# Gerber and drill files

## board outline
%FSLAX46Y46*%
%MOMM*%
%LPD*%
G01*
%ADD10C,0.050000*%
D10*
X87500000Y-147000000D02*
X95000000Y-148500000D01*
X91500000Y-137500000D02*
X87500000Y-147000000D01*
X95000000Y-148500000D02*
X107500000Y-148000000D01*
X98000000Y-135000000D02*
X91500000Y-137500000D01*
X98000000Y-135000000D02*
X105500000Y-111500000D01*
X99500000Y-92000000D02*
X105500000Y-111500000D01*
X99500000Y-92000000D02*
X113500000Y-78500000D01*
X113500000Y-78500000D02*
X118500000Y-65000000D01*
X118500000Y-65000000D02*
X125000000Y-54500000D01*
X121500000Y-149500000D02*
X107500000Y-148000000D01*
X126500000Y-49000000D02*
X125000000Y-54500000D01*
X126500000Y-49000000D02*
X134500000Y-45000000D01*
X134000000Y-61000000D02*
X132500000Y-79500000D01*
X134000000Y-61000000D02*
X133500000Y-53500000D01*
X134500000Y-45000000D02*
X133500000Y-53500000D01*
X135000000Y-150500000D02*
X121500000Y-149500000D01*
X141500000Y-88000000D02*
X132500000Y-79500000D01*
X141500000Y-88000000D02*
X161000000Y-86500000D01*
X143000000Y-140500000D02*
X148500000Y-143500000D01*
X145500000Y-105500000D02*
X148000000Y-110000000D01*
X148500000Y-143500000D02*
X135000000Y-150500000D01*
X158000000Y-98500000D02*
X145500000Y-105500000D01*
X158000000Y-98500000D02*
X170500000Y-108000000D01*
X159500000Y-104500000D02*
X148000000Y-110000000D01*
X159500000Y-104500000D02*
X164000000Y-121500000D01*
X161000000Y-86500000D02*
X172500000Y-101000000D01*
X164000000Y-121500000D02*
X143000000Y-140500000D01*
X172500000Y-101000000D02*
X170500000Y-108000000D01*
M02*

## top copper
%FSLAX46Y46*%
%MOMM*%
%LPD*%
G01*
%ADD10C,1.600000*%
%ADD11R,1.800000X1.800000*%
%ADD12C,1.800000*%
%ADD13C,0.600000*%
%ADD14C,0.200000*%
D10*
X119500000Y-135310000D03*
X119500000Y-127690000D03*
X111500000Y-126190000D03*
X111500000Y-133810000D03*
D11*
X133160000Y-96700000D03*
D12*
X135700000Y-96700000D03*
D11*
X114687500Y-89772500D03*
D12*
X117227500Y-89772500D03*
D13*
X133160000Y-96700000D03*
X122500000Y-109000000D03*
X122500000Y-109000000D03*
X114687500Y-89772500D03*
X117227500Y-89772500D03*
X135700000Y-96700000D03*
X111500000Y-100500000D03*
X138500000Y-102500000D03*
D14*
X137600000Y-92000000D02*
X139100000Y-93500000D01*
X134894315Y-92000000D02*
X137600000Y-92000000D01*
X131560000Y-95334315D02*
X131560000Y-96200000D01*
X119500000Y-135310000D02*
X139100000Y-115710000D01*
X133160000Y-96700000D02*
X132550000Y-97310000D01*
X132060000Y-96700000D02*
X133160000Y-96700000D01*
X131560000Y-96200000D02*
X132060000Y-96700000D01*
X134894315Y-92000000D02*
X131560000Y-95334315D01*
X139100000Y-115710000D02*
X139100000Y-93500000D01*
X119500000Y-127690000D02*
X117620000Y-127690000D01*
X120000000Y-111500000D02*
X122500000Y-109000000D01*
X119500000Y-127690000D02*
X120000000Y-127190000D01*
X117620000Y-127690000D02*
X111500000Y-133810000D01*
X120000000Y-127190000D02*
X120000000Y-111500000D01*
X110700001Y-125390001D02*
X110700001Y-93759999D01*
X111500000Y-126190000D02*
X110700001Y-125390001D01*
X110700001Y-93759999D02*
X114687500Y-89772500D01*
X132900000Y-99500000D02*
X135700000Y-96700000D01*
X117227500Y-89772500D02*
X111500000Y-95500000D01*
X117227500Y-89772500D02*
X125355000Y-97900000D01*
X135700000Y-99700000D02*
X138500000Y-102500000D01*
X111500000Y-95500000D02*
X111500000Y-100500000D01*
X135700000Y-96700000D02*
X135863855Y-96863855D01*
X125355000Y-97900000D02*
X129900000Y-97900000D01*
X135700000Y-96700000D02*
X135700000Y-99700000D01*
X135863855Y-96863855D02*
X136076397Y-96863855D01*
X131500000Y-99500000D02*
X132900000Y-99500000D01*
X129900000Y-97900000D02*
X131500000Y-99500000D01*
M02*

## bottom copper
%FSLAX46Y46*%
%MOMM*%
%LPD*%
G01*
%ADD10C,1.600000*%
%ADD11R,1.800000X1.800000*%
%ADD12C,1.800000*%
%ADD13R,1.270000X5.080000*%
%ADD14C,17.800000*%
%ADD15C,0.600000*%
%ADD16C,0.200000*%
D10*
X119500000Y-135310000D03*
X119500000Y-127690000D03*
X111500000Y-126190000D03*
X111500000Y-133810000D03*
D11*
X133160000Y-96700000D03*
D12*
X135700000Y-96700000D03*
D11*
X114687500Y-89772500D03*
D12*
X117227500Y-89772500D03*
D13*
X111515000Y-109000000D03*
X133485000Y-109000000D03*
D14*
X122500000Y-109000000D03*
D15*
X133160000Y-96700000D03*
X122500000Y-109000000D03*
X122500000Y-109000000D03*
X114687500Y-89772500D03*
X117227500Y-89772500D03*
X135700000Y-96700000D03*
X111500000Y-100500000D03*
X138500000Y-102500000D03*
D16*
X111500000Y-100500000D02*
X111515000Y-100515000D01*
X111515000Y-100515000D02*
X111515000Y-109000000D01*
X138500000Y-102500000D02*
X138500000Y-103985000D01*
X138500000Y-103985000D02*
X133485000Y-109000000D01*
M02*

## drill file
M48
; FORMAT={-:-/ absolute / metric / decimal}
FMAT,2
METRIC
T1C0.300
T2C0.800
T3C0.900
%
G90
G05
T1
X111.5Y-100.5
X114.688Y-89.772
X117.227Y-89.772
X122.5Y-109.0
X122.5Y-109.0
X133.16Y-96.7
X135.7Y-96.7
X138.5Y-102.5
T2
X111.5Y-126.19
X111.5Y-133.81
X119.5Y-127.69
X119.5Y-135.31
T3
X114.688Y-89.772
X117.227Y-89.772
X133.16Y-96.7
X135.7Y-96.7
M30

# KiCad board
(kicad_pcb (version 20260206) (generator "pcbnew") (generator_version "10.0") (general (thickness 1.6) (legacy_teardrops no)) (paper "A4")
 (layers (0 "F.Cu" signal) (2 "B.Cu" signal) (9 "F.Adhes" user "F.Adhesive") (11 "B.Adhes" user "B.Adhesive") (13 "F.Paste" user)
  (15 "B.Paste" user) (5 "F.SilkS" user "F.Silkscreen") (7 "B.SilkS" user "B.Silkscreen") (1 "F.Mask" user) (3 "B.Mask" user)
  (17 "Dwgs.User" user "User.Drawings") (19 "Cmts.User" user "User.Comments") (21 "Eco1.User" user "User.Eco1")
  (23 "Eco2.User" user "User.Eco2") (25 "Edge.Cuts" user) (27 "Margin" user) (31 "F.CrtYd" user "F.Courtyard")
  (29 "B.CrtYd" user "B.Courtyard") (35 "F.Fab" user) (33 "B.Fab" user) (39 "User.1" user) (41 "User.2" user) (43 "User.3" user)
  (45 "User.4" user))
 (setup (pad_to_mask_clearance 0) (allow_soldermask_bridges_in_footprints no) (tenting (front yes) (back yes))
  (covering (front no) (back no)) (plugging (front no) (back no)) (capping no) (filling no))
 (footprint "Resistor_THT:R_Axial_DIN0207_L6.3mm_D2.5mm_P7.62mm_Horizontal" (layer "F.Cu") (at 119.5 135.31 90)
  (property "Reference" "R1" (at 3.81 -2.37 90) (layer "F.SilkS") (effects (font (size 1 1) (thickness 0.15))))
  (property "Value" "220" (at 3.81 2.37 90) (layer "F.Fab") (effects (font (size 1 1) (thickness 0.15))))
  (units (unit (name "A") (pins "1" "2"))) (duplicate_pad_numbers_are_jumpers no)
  (pad "1" thru_hole circle (at 0 0 90) (size 1.6 1.6) (drill 0.8) (layers "*.Cu" "*.Mask") (remove_unused_layers no) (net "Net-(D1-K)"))
  (pad "2" thru_hole circle (at 7.62 0 90) (size 1.6 1.6) (drill 0.8) (layers "*.Cu" "*.Mask") (remove_unused_layers no) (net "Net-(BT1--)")))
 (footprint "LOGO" (layer "F.Cu") (at 130 97.5)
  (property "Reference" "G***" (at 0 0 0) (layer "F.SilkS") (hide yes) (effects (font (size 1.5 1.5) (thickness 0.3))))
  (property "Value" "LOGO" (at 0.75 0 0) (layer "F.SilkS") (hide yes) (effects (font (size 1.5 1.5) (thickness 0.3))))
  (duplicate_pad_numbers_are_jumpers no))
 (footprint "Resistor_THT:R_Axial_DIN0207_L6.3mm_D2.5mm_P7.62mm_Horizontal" (layer "F.Cu") (at 111.5 126.19 -90)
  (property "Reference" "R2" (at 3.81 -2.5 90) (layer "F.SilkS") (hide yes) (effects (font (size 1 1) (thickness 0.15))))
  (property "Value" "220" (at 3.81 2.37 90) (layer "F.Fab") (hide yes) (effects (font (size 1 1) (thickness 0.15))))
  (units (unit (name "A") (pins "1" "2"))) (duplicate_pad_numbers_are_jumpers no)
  (pad "1" thru_hole circle (at 0 0 270) (size 1.6 1.6) (drill 0.8) (layers "*.Cu" "*.Mask") (remove_unused_layers no) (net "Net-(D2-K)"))
  (pad "2" thru_hole circle (at 7.62 0 270) (size 1.6 1.6) (drill 0.8) (layers "*.Cu" "*.Mask") (remove_unused_layers no)
   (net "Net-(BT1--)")))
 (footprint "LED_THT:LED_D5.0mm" (layer "F.Cu") (at 133.16 96.7)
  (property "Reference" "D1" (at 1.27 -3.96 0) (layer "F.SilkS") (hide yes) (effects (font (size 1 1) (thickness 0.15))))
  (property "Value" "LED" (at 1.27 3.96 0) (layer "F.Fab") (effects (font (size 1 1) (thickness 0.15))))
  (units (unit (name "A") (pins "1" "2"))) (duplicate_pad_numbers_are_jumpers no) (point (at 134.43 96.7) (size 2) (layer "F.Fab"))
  (pad "1" thru_hole rect (at 0 0) (size 1.8 1.8) (drill 0.9) (layers "*.Cu" "*.Mask") (remove_unused_layers no) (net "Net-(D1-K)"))
  (pad "2" thru_hole circle (at 2.54 0) (size 1.8 1.8) (drill 0.9) (layers "*.Cu" "*.Mask") (remove_unused_layers no) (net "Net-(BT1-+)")))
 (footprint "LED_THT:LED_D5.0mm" (layer "F.Cu") (at 114.6875 89.7725)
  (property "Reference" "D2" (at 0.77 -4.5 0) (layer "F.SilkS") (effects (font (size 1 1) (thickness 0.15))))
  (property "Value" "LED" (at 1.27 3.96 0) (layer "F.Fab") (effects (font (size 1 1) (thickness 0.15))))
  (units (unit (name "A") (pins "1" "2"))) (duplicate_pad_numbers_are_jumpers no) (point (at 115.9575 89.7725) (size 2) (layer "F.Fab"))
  (pad "1" thru_hole rect (at 0 0) (size 1.8 1.8) (drill 0.9) (layers "*.Cu" "*.Mask") (remove_unused_layers no) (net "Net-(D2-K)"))
  (pad "2" thru_hole circle (at 2.54 0) (size 1.8 1.8) (drill 0.9) (layers "*.Cu" "*.Mask") (remove_unused_layers no) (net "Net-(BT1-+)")))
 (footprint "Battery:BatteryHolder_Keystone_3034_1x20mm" (layer "B.Cu") (at 122.5 109)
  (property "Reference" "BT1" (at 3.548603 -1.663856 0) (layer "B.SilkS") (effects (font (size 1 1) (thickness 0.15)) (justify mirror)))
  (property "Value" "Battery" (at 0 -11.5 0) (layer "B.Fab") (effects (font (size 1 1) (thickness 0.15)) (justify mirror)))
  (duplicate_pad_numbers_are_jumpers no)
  (pad "1" smd rect (at -10.985 0) (size 1.27 5.08) (layers "B.Cu" "B.Mask" "B.Paste") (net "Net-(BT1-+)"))
  (pad "1" smd rect (at 10.985 0) (size 1.27 5.08) (layers "B.Cu" "B.Mask" "B.Paste") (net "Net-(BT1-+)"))
  (pad "2" smd circle (at 0 0) (size 17.8 17.8) (layers "B.Cu" "B.Mask") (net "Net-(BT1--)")))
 (gr_line (start 87.5 147) (end 95 148.5) (stroke (width 0.05) (type default)) (layer "Edge.Cuts"))
 (gr_line (start 91.5 137.5) (end 87.5 147) (stroke (width 0.05) (type default)) (layer "Edge.Cuts"))
 (gr_line (start 95 148.5) (end 107.5 148) (stroke (width 0.05) (type default)) (layer "Edge.Cuts"))
 (gr_line (start 98 135) (end 91.5 137.5) (stroke (width 0.05) (type default)) (layer "Edge.Cuts"))
 (gr_line (start 98 135) (end 105.5 111.5) (stroke (width 0.05) (type default)) (layer "Edge.Cuts"))
 (gr_line (start 99.5 92) (end 105.5 111.5) (stroke (width 0.05) (type default)) (layer "Edge.Cuts"))
 (gr_line (start 99.5 92) (end 113.5 78.5) (stroke (width 0.05) (type default)) (layer "Edge.Cuts"))
 (gr_line (start 113.5 78.5) (end 118.5 65) (stroke (width 0.05) (type default)) (layer "Edge.Cuts"))
 (gr_line (start 118.5 65) (end 125 54.5) (stroke (width 0.05) (type default)) (layer "Edge.Cuts"))
 (gr_line (start 121.5 149.5) (end 107.5 148) (stroke (width 0.05) (type default)) (layer "Edge.Cuts"))
 (gr_line (start 126.5 49) (end 125 54.5) (stroke (width 0.05) (type default)) (layer "Edge.Cuts"))
 (gr_line (start 126.5 49) (end 134.5 45) (stroke (width 0.05) (type default)) (layer "Edge.Cuts"))
 (gr_line (start 134 61) (end 132.5 79.5) (stroke (width 0.05) (type default)) (layer "Edge.Cuts"))
 (gr_line (start 134 61) (end 133.5 53.5) (stroke (width 0.05) (type default)) (layer "Edge.Cuts"))
 (gr_line (start 134.5 45) (end 133.5 53.5) (stroke (width 0.05) (type default)) (layer "Edge.Cuts"))
 (gr_line (start 135 150.5) (end 121.5 149.5) (stroke (width 0.05) (type default)) (layer "Edge.Cuts"))
 (gr_line (start 141.5 88) (end 132.5 79.5) (stroke (width 0.05) (type default)) (layer "Edge.Cuts"))
 (gr_line (start 141.5 88) (end 161 86.5) (stroke (width 0.05) (type default)) (layer "Edge.Cuts"))
 (gr_line (start 143 140.5) (end 148.5 143.5) (stroke (width 0.05) (type default)) (layer "Edge.Cuts"))
 (gr_line (start 145.5 105.5) (end 148 110) (stroke (width 0.05) (type default)) (layer "Edge.Cuts"))
 (gr_line (start 148.5 143.5) (end 135 150.5) (stroke (width 0.05) (type default)) (layer "Edge.Cuts"))
 (gr_line (start 158 98.5) (end 145.5 105.5) (stroke (width 0.05) (type default)) (layer "Edge.Cuts"))
 (gr_line (start 158 98.5) (end 170.5 108) (stroke (width 0.05) (type default)) (layer "Edge.Cuts"))
 (gr_line (start 159.5 104.5) (end 148 110) (stroke (width 0.05) (type default)) (layer "Edge.Cuts"))
 (gr_line (start 159.5 104.5) (end 164 121.5) (stroke (width 0.05) (type default)) (layer "Edge.Cuts"))
 (gr_line (start 161 86.5) (end 172.5 101) (stroke (width 0.05) (type default)) (layer "Edge.Cuts"))
 (gr_line (start 164 121.5) (end 143 140.5) (stroke (width 0.05) (type default)) (layer "Edge.Cuts"))
 (gr_line (start 172.5 101) (end 170.5 108) (stroke (width 0.05) (type default)) (layer "Edge.Cuts"))
 (segment (start 137.6 92) (end 139.1 93.5) (width 0.2) (layer "F.Cu") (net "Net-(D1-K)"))
 (segment (start 134.894315 92) (end 137.6 92) (width 0.2) (layer "F.Cu") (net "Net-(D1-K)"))
 (segment (start 131.56 95.334315) (end 131.56 96.2) (width 0.2) (layer "F.Cu") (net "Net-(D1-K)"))
 (segment (start 119.5 135.31) (end 139.1 115.71) (width 0.2) (layer "F.Cu") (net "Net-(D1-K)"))
 (segment (start 133.16 96.7) (end 132.55 97.31) (width 0.2) (layer "F.Cu") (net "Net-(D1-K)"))
 (segment (start 132.06 96.7) (end 133.16 96.7) (width 0.2) (layer "F.Cu") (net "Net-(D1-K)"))
 (segment (start 131.56 96.2) (end 132.06 96.7) (width 0.2) (layer "F.Cu") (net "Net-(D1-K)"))
 (segment (start 134.894315 92) (end 131.56 95.334315) (width 0.2) (layer "F.Cu") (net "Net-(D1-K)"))
 (segment (start 139.1 115.71) (end 139.1 93.5) (width 0.2) (layer "F.Cu") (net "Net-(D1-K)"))
 (via (at 133.16 96.7) (size 0.6) (drill 0.3) (layers "F.Cu" "B.Cu") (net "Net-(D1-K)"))
 (segment (start 119.5 127.69) (end 117.62 127.69) (width 0.2) (layer "F.Cu") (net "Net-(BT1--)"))
 (segment (start 120 111.5) (end 122.5 109) (width 0.2) (layer "F.Cu") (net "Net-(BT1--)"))
 (segment (start 119.5 127.69) (end 120 127.19) (width 0.2) (layer "F.Cu") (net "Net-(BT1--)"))
 (segment (start 117.62 127.69) (end 111.5 133.81) (width 0.2) (layer "F.Cu") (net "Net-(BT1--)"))
 (segment (start 120 127.19) (end 120 111.5) (width 0.2) (layer "F.Cu") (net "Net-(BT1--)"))
 (via (at 122.5 109) (size 0.6) (drill 0.3) (layers "F.Cu" "B.Cu") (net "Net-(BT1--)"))
 (via (at 122.5 109) (size 0.6) (drill 0.3) (layers "F.Cu" "B.Cu") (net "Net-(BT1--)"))
 (segment (start 110.700001 125.390001) (end 110.700001 93.759999) (width 0.2) (layer "F.Cu") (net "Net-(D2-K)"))
 (segment (start 111.5 126.19) (end 110.700001 125.390001) (width 0.2) (layer "F.Cu") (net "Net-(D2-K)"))
 (segment (start 110.700001 93.759999) (end 114.6875 89.7725) (width 0.2) (layer "F.Cu") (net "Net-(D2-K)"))
 (via (at 114.6875 89.7725) (size 0.6) (drill 0.3) (layers "F.Cu" "B.Cu") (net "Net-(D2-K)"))
 (segment (start 132.9 99.5) (end 135.7 96.7) (width 0.2) (layer "F.Cu") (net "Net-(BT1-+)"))
 (segment (start 117.2275 89.7725) (end 111.5 95.5) (width 0.2) (layer "F.Cu") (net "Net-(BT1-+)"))
 (segment (start 117.2275 89.7725) (end 125.355 97.9) (width 0.2) (layer "F.Cu") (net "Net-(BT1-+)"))
 (segment (start 135.7 99.7) (end 138.5 102.5) (width 0.2) (layer "F.Cu") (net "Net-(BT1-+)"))
 (segment (start 111.5 95.5) (end 111.5 100.5) (width 0.2) (layer "F.Cu") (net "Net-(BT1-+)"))
 (segment (start 135.7 96.7) (end 135.863855 96.863855) (width 0.2) (layer "F.Cu") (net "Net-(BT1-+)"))
 (segment (start 125.355 97.9) (end 129.9 97.9) (width 0.2) (layer "F.Cu") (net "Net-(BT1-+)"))
 (segment (start 135.7 96.7) (end 135.7 99.7) (width 0.2) (layer "F.Cu") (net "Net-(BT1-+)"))
 (segment (start 135.863855 96.863855) (end 136.076397 96.863855) (width 0.2) (layer "F.Cu") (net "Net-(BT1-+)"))
 (segment (start 131.5 99.5) (end 132.9 99.5) (width 0.2) (layer "F.Cu") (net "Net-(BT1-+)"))
 (segment (start 129.9 97.9) (end 131.5 99.5) (width 0.2) (layer "F.Cu") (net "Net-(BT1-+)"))
 (via (at 117.2275 89.7725) (size 0.6) (drill 0.3) (layers "F.Cu" "B.Cu") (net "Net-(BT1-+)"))
 (via (at 135.7 96.7) (size 0.6) (drill 0.3) (layers "F.Cu" "B.Cu") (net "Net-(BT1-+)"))
 (via (at 111.5 100.5) (size 0.6) (drill 0.3) (layers "F.Cu" "B.Cu") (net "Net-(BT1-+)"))
 (via (at 138.5 102.5) (size 0.6) (drill 0.3) (layers "F.Cu" "B.Cu") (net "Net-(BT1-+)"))
 (segment (start 111.5 100.5) (end 111.515 100.515) (width 0.2) (layer "B.Cu") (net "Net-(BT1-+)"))
 (segment (start 111.515 100.515) (end 111.515 109) (width 0.2) (layer "B.Cu") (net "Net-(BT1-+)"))
 (segment (start 138.5 102.5) (end 138.5 103.985) (width 0.2) (layer "B.Cu") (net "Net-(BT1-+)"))
 (segment (start 138.5 103.985) (end 133.485 109) (width 0.2) (layer "B.Cu") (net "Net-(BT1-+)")))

